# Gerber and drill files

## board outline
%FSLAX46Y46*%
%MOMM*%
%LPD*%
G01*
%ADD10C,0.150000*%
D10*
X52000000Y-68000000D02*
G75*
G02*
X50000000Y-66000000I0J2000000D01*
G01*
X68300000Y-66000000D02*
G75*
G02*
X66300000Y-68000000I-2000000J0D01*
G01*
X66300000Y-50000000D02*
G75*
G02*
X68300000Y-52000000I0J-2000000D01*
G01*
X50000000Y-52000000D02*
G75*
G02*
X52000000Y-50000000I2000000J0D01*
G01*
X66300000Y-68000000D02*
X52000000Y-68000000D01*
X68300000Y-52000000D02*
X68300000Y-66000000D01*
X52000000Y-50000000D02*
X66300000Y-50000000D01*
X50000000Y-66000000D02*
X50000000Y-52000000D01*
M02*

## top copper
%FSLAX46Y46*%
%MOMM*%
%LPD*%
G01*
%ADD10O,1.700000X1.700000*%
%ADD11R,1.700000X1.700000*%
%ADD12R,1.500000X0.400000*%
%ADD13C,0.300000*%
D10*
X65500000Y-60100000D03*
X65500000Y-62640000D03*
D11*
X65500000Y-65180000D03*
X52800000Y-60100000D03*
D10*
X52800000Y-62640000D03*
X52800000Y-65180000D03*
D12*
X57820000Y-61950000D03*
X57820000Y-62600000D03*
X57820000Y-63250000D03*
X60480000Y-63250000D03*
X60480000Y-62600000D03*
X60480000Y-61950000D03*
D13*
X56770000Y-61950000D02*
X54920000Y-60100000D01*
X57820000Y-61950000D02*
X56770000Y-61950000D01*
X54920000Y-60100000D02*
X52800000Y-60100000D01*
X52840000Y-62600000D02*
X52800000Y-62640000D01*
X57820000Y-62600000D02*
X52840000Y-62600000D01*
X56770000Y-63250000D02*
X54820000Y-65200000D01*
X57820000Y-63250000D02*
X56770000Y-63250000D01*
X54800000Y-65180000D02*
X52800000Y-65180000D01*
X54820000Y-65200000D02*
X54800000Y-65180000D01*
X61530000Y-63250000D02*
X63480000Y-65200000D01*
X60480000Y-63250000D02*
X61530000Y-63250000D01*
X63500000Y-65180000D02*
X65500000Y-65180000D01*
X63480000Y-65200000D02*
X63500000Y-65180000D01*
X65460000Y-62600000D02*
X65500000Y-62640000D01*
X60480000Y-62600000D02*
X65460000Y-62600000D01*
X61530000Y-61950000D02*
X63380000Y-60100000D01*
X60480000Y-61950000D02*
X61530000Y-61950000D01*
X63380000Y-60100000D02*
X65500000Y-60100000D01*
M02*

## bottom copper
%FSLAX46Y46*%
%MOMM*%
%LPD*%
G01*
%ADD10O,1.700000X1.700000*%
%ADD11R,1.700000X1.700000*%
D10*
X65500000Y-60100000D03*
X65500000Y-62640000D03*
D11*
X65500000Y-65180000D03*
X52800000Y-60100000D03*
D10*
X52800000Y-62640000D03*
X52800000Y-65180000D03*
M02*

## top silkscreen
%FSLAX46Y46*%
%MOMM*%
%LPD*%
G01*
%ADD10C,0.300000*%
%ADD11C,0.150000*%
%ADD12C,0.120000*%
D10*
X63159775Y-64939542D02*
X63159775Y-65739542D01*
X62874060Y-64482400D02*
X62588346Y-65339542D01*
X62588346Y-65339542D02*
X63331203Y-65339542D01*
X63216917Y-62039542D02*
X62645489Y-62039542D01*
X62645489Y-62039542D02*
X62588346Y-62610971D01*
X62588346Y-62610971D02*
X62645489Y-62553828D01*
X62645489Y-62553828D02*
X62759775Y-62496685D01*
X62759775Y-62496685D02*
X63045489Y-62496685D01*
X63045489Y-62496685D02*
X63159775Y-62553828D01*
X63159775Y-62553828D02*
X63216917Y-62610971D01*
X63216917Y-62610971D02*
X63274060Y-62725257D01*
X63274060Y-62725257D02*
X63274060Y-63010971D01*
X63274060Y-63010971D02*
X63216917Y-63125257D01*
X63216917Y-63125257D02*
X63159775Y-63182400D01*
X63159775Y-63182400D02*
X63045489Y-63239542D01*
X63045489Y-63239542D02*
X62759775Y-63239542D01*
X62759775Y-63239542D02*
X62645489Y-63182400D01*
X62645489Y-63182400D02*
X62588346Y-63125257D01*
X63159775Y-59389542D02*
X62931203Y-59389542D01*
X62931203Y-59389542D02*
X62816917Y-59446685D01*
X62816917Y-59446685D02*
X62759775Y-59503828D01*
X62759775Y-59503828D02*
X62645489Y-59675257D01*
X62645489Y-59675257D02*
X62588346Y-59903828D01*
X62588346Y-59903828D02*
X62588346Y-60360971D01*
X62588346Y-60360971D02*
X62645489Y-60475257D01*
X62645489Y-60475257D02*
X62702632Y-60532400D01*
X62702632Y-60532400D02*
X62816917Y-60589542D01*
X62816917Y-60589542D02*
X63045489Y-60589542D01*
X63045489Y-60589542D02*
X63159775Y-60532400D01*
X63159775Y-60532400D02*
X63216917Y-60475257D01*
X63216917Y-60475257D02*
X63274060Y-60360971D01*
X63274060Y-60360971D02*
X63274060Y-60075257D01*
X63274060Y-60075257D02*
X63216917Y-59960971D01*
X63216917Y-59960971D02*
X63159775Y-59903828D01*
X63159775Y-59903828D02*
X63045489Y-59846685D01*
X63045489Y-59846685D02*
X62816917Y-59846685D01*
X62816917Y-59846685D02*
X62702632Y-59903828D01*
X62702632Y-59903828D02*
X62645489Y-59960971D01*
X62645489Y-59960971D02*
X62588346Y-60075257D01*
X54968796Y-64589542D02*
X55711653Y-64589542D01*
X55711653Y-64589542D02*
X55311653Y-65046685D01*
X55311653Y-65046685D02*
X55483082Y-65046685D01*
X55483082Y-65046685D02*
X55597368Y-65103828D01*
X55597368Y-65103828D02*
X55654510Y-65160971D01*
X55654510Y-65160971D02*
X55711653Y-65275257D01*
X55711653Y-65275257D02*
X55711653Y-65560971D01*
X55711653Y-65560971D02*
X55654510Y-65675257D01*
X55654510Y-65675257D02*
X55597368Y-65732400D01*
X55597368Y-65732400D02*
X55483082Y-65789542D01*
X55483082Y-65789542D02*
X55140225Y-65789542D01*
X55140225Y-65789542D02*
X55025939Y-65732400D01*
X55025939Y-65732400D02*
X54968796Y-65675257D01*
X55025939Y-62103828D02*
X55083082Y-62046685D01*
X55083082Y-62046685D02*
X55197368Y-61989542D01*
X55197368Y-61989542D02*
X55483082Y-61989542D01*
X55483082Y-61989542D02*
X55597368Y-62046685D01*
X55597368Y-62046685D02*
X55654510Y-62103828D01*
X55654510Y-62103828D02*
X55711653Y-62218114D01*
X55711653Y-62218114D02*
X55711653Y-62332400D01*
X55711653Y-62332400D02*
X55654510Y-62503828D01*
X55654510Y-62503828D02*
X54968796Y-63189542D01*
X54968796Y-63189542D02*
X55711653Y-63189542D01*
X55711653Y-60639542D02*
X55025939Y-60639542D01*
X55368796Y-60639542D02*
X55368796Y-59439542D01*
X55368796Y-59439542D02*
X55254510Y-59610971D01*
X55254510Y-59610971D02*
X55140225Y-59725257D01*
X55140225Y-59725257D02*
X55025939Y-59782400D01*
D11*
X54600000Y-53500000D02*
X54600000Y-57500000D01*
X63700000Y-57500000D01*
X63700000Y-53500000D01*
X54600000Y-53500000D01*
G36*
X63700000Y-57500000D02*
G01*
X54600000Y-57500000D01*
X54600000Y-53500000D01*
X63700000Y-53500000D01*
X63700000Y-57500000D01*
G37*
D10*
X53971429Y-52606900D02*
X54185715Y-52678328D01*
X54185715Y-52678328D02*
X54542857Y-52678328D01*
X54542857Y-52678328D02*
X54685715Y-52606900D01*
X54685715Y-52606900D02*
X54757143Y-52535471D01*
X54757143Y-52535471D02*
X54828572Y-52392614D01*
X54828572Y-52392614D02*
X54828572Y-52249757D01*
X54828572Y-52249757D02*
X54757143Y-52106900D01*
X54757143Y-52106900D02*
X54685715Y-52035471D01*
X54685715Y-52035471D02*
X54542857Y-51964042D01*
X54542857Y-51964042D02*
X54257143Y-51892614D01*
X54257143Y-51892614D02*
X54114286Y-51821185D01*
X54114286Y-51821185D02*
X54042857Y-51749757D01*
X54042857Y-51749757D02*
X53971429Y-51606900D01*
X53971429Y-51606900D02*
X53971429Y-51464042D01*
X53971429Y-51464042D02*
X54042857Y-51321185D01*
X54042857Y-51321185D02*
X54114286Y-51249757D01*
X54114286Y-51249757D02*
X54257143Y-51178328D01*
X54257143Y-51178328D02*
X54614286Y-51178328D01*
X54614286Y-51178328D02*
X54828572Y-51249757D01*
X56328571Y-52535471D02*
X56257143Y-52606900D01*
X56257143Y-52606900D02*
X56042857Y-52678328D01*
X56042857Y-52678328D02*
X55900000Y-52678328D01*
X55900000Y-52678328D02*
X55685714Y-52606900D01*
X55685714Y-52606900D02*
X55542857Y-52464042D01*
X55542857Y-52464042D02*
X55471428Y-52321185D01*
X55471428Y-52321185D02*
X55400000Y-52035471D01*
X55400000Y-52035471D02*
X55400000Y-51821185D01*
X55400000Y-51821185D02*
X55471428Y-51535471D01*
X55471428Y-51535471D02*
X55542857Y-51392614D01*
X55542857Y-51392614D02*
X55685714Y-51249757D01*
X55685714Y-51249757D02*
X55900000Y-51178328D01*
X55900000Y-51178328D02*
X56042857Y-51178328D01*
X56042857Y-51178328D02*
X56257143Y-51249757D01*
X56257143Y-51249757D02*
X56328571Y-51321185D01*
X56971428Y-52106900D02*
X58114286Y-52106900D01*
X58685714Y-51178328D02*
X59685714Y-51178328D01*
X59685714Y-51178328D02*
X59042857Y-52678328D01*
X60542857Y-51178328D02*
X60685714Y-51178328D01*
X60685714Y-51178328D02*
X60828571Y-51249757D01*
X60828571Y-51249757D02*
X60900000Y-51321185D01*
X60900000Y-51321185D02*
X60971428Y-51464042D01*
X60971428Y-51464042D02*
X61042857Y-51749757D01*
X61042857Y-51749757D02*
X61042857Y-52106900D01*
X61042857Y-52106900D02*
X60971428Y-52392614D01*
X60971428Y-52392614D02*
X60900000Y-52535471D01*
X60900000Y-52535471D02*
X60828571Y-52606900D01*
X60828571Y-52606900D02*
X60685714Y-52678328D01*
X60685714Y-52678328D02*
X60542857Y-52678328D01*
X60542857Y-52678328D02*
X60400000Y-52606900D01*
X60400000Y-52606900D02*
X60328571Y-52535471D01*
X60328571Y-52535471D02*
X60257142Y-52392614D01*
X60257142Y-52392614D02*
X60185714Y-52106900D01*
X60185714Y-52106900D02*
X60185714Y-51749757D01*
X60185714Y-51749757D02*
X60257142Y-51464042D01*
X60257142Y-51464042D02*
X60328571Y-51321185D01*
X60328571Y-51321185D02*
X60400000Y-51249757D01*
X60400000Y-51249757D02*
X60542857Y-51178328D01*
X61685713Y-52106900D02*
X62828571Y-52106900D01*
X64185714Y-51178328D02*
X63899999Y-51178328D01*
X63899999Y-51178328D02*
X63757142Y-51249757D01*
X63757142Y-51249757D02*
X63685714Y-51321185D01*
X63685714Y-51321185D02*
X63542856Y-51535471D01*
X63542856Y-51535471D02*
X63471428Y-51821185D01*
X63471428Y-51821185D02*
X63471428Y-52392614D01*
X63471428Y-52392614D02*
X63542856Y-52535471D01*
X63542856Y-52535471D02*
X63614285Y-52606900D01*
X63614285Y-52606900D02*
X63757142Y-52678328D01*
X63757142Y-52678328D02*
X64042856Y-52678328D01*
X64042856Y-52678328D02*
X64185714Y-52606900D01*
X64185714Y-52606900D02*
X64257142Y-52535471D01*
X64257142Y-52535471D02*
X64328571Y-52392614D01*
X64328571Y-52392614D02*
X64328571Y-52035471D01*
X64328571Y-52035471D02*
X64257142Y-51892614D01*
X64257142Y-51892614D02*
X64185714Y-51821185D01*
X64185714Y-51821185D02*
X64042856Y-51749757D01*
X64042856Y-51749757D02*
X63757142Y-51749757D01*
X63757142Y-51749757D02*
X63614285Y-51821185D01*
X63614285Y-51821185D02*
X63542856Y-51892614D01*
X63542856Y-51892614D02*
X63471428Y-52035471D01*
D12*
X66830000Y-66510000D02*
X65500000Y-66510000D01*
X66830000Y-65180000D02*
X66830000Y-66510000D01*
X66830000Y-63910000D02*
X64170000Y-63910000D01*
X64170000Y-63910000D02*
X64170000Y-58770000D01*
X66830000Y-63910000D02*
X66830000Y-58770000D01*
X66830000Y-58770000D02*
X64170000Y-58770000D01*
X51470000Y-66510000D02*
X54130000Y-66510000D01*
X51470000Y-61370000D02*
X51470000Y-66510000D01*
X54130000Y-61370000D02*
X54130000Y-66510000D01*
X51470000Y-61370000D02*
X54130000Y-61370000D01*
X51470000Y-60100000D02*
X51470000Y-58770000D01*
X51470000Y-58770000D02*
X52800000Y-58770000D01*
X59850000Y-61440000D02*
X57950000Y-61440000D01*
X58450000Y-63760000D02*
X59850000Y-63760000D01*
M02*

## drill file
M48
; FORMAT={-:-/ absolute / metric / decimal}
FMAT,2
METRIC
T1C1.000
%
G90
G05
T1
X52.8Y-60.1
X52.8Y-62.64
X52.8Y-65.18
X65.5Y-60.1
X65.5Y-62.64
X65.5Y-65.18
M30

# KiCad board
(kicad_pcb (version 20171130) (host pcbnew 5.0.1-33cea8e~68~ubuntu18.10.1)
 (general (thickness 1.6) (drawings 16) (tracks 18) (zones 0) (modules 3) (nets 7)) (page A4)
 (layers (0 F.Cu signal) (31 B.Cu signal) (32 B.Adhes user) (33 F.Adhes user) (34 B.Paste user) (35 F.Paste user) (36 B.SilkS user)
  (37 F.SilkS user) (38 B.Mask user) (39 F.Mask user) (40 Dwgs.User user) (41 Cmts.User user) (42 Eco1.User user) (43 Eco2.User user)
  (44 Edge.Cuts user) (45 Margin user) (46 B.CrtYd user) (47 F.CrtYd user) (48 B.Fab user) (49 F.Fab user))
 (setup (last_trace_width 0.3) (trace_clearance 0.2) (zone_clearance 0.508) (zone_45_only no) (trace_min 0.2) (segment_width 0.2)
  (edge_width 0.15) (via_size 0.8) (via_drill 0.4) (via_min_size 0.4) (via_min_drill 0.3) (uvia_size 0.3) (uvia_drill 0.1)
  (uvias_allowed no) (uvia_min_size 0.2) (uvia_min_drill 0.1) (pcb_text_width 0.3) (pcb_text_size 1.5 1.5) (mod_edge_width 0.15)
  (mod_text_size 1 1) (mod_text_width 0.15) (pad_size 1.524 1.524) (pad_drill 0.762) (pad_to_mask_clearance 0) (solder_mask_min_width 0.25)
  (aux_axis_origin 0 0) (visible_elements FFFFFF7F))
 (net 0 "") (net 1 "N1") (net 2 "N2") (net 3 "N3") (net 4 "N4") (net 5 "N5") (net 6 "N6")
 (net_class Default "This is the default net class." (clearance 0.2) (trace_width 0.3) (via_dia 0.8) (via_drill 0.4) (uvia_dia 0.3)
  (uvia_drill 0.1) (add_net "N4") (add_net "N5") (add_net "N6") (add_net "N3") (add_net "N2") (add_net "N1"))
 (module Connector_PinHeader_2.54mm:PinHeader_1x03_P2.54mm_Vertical (layer F.Cu) (at 65.5 65.18 180)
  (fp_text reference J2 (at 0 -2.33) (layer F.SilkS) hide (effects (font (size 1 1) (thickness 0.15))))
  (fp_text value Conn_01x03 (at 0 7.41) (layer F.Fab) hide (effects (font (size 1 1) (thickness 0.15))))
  (fp_line (start -1.33 -1.33) (end 0 -1.33) (layer F.SilkS) (width 0.12))
  (fp_line (start -1.33 0) (end -1.33 -1.33) (layer F.SilkS) (width 0.12))
  (fp_line (start -1.33 1.27) (end 1.33 1.27) (layer F.SilkS) (width 0.12))
  (fp_line (start 1.33 1.27) (end 1.33 6.41) (layer F.SilkS) (width 0.12))
  (fp_line (start -1.33 1.27) (end -1.33 6.41) (layer F.SilkS) (width 0.12))
  (fp_line (start -1.33 6.41) (end 1.33 6.41) (layer F.SilkS) (width 0.12))
  (pad 3 thru_hole oval (at 0 5.08) (size 1.7 1.7) (drill 1) (layers *.Cu *.Mask) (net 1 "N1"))
  (pad 2 thru_hole oval (at 0 2.54) (size 1.7 1.7) (drill 1) (layers *.Cu *.Mask) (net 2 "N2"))
  (pad 1 thru_hole rect (at 0 0) (size 1.7 1.7) (drill 1) (layers *.Cu *.Mask) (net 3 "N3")))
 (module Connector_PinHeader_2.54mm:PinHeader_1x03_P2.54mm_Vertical (layer F.Cu) (at 52.8 60.1)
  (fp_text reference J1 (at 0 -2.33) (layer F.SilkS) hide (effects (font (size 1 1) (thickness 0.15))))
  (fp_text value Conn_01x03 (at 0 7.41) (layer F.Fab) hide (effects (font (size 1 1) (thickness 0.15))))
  (fp_line (start -1.33 6.41) (end 1.33 6.41) (layer F.SilkS) (width 0.12))
  (fp_line (start -1.33 1.27) (end -1.33 6.41) (layer F.SilkS) (width 0.12))
  (fp_line (start 1.33 1.27) (end 1.33 6.41) (layer F.SilkS) (width 0.12))
  (fp_line (start -1.33 1.27) (end 1.33 1.27) (layer F.SilkS) (width 0.12))
  (fp_line (start -1.33 0) (end -1.33 -1.33) (layer F.SilkS) (width 0.12))
  (fp_line (start -1.33 -1.33) (end 0 -1.33) (layer F.SilkS) (width 0.12))
  (pad 1 thru_hole rect (at 0 0) (size 1.7 1.7) (drill 1) (layers *.Cu *.Mask) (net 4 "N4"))
  (pad 2 thru_hole oval (at 0 2.54) (size 1.7 1.7) (drill 1) (layers *.Cu *.Mask) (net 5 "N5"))
  (pad 3 thru_hole oval (at 0 5.08) (size 1.7 1.7) (drill 1) (layers *.Cu *.Mask) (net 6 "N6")))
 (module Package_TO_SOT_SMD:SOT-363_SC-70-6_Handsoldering (layer F.Cu) (at 59.15 62.6)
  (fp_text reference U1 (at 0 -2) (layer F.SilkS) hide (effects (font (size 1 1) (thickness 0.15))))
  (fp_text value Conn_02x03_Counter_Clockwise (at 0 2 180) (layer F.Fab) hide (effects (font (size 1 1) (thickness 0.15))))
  (fp_line (start 0.7 -1.16) (end -1.2 -1.16) (layer F.SilkS) (width 0.12))
  (fp_line (start -0.7 1.16) (end 0.7 1.16) (layer F.SilkS) (width 0.12))
  (pad 1 smd rect (at -1.33 -0.65) (size 1.5 0.4) (layers F.Cu F.Paste F.Mask) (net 4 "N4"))
  (pad 2 smd rect (at -1.33 0) (size 1.5 0.4) (layers F.Cu F.Paste F.Mask) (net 5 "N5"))
  (pad 3 smd rect (at -1.33 0.65) (size 1.5 0.4) (layers F.Cu F.Paste F.Mask) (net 6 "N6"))
  (pad 4 smd rect (at 1.33 0.65) (size 1.5 0.4) (layers F.Cu F.Paste F.Mask) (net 3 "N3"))
  (pad 5 smd rect (at 1.33 0) (size 1.5 0.4) (layers F.Cu F.Paste F.Mask) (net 2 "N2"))
  (pad 6 smd rect (at 1.33 -0.65) (size 1.5 0.4) (layers F.Cu F.Paste F.Mask) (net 1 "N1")))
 (gr_arc (start 52 66) (end 50 66) (angle -90) (layer Edge.Cuts) (width 0.15))
 (gr_arc (start 66.3 66) (end 66.3 68) (angle -90) (layer Edge.Cuts) (width 0.15))
 (gr_arc (start 66.3 52) (end 68.3 52) (angle -90) (layer Edge.Cuts) (width 0.15))
 (gr_arc (start 52 52) (end 52 50) (angle -90) (layer Edge.Cuts) (width 0.15))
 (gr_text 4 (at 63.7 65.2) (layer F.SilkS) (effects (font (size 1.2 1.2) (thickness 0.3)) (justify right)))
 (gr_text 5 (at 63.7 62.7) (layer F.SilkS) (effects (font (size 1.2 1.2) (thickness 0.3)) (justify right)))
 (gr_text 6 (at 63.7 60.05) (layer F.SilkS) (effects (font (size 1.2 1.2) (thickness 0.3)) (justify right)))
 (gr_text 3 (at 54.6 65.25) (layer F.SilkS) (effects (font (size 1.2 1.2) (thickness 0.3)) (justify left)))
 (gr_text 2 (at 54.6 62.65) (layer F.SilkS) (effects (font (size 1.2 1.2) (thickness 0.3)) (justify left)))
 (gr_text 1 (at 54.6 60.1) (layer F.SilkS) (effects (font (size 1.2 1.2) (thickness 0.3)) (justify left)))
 (gr_line (start 66.3 68) (end 52 68) (layer Edge.Cuts) (width 0.15))
 (gr_poly (pts (xy 54.6 53.5) (xy 54.6 57.5) (xy 63.7 57.5) (xy 63.7 53.5)) (layer F.SilkS) (width 0.15))
 (gr_line (start 68.3 52) (end 68.3 66) (layer Edge.Cuts) (width 0.15))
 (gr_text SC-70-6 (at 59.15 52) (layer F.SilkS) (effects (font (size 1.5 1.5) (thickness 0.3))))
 (gr_line (start 52 50) (end 66.3 50) (layer Edge.Cuts) (width 0.15))
 (gr_line (start 50 66) (end 50 52) (layer Edge.Cuts) (width 0.15))
 (segment (start 56.77 61.95) (end 54.92 60.1) (width 0.3) (layer F.Cu) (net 4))
 (segment (start 57.82 61.95) (end 56.77 61.95) (width 0.3) (layer F.Cu) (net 4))
 (segment (start 54.92 60.1) (end 52.8 60.1) (width 0.3) (layer F.Cu) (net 4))
 (segment (start 52.84 62.6) (end 52.8 62.64) (width 0.3) (layer F.Cu) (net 5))
 (segment (start 57.82 62.6) (end 52.84 62.6) (width 0.3) (layer F.Cu) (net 5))
 (segment (start 56.77 63.25) (end 54.82 65.2) (width 0.3) (layer F.Cu) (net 6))
 (segment (start 57.82 63.25) (end 56.77 63.25) (width 0.3) (layer F.Cu) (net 6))
 (segment (start 54.8 65.18) (end 52.8 65.18) (width 0.3) (layer F.Cu) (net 6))
 (segment (start 54.82 65.2) (end 54.8 65.18) (width 0.3) (layer F.Cu) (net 6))
 (segment (start 61.53 63.25) (end 63.48 65.2) (width 0.3) (layer F.Cu) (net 3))
 (segment (start 60.48 63.25) (end 61.53 63.25) (width 0.3) (layer F.Cu) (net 3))
 (segment (start 63.5 65.18) (end 65.5 65.18) (width 0.3) (layer F.Cu) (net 3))
 (segment (start 63.48 65.2) (end 63.5 65.18) (width 0.3) (layer F.Cu) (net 3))
 (segment (start 65.46 62.6) (end 65.5 62.64) (width 0.3) (layer F.Cu) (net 2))
 (segment (start 60.48 62.6) (end 65.46 62.6) (width 0.3) (layer F.Cu) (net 2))
 (segment (start 61.53 61.95) (end 63.38 60.1) (width 0.3) (layer F.Cu) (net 1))
 (segment (start 60.48 61.95) (end 61.53 61.95) (width 0.3) (layer F.Cu) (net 1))
 (segment (start 63.38 60.1) (end 65.5 60.1) (width 0.3) (layer F.Cu) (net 1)))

